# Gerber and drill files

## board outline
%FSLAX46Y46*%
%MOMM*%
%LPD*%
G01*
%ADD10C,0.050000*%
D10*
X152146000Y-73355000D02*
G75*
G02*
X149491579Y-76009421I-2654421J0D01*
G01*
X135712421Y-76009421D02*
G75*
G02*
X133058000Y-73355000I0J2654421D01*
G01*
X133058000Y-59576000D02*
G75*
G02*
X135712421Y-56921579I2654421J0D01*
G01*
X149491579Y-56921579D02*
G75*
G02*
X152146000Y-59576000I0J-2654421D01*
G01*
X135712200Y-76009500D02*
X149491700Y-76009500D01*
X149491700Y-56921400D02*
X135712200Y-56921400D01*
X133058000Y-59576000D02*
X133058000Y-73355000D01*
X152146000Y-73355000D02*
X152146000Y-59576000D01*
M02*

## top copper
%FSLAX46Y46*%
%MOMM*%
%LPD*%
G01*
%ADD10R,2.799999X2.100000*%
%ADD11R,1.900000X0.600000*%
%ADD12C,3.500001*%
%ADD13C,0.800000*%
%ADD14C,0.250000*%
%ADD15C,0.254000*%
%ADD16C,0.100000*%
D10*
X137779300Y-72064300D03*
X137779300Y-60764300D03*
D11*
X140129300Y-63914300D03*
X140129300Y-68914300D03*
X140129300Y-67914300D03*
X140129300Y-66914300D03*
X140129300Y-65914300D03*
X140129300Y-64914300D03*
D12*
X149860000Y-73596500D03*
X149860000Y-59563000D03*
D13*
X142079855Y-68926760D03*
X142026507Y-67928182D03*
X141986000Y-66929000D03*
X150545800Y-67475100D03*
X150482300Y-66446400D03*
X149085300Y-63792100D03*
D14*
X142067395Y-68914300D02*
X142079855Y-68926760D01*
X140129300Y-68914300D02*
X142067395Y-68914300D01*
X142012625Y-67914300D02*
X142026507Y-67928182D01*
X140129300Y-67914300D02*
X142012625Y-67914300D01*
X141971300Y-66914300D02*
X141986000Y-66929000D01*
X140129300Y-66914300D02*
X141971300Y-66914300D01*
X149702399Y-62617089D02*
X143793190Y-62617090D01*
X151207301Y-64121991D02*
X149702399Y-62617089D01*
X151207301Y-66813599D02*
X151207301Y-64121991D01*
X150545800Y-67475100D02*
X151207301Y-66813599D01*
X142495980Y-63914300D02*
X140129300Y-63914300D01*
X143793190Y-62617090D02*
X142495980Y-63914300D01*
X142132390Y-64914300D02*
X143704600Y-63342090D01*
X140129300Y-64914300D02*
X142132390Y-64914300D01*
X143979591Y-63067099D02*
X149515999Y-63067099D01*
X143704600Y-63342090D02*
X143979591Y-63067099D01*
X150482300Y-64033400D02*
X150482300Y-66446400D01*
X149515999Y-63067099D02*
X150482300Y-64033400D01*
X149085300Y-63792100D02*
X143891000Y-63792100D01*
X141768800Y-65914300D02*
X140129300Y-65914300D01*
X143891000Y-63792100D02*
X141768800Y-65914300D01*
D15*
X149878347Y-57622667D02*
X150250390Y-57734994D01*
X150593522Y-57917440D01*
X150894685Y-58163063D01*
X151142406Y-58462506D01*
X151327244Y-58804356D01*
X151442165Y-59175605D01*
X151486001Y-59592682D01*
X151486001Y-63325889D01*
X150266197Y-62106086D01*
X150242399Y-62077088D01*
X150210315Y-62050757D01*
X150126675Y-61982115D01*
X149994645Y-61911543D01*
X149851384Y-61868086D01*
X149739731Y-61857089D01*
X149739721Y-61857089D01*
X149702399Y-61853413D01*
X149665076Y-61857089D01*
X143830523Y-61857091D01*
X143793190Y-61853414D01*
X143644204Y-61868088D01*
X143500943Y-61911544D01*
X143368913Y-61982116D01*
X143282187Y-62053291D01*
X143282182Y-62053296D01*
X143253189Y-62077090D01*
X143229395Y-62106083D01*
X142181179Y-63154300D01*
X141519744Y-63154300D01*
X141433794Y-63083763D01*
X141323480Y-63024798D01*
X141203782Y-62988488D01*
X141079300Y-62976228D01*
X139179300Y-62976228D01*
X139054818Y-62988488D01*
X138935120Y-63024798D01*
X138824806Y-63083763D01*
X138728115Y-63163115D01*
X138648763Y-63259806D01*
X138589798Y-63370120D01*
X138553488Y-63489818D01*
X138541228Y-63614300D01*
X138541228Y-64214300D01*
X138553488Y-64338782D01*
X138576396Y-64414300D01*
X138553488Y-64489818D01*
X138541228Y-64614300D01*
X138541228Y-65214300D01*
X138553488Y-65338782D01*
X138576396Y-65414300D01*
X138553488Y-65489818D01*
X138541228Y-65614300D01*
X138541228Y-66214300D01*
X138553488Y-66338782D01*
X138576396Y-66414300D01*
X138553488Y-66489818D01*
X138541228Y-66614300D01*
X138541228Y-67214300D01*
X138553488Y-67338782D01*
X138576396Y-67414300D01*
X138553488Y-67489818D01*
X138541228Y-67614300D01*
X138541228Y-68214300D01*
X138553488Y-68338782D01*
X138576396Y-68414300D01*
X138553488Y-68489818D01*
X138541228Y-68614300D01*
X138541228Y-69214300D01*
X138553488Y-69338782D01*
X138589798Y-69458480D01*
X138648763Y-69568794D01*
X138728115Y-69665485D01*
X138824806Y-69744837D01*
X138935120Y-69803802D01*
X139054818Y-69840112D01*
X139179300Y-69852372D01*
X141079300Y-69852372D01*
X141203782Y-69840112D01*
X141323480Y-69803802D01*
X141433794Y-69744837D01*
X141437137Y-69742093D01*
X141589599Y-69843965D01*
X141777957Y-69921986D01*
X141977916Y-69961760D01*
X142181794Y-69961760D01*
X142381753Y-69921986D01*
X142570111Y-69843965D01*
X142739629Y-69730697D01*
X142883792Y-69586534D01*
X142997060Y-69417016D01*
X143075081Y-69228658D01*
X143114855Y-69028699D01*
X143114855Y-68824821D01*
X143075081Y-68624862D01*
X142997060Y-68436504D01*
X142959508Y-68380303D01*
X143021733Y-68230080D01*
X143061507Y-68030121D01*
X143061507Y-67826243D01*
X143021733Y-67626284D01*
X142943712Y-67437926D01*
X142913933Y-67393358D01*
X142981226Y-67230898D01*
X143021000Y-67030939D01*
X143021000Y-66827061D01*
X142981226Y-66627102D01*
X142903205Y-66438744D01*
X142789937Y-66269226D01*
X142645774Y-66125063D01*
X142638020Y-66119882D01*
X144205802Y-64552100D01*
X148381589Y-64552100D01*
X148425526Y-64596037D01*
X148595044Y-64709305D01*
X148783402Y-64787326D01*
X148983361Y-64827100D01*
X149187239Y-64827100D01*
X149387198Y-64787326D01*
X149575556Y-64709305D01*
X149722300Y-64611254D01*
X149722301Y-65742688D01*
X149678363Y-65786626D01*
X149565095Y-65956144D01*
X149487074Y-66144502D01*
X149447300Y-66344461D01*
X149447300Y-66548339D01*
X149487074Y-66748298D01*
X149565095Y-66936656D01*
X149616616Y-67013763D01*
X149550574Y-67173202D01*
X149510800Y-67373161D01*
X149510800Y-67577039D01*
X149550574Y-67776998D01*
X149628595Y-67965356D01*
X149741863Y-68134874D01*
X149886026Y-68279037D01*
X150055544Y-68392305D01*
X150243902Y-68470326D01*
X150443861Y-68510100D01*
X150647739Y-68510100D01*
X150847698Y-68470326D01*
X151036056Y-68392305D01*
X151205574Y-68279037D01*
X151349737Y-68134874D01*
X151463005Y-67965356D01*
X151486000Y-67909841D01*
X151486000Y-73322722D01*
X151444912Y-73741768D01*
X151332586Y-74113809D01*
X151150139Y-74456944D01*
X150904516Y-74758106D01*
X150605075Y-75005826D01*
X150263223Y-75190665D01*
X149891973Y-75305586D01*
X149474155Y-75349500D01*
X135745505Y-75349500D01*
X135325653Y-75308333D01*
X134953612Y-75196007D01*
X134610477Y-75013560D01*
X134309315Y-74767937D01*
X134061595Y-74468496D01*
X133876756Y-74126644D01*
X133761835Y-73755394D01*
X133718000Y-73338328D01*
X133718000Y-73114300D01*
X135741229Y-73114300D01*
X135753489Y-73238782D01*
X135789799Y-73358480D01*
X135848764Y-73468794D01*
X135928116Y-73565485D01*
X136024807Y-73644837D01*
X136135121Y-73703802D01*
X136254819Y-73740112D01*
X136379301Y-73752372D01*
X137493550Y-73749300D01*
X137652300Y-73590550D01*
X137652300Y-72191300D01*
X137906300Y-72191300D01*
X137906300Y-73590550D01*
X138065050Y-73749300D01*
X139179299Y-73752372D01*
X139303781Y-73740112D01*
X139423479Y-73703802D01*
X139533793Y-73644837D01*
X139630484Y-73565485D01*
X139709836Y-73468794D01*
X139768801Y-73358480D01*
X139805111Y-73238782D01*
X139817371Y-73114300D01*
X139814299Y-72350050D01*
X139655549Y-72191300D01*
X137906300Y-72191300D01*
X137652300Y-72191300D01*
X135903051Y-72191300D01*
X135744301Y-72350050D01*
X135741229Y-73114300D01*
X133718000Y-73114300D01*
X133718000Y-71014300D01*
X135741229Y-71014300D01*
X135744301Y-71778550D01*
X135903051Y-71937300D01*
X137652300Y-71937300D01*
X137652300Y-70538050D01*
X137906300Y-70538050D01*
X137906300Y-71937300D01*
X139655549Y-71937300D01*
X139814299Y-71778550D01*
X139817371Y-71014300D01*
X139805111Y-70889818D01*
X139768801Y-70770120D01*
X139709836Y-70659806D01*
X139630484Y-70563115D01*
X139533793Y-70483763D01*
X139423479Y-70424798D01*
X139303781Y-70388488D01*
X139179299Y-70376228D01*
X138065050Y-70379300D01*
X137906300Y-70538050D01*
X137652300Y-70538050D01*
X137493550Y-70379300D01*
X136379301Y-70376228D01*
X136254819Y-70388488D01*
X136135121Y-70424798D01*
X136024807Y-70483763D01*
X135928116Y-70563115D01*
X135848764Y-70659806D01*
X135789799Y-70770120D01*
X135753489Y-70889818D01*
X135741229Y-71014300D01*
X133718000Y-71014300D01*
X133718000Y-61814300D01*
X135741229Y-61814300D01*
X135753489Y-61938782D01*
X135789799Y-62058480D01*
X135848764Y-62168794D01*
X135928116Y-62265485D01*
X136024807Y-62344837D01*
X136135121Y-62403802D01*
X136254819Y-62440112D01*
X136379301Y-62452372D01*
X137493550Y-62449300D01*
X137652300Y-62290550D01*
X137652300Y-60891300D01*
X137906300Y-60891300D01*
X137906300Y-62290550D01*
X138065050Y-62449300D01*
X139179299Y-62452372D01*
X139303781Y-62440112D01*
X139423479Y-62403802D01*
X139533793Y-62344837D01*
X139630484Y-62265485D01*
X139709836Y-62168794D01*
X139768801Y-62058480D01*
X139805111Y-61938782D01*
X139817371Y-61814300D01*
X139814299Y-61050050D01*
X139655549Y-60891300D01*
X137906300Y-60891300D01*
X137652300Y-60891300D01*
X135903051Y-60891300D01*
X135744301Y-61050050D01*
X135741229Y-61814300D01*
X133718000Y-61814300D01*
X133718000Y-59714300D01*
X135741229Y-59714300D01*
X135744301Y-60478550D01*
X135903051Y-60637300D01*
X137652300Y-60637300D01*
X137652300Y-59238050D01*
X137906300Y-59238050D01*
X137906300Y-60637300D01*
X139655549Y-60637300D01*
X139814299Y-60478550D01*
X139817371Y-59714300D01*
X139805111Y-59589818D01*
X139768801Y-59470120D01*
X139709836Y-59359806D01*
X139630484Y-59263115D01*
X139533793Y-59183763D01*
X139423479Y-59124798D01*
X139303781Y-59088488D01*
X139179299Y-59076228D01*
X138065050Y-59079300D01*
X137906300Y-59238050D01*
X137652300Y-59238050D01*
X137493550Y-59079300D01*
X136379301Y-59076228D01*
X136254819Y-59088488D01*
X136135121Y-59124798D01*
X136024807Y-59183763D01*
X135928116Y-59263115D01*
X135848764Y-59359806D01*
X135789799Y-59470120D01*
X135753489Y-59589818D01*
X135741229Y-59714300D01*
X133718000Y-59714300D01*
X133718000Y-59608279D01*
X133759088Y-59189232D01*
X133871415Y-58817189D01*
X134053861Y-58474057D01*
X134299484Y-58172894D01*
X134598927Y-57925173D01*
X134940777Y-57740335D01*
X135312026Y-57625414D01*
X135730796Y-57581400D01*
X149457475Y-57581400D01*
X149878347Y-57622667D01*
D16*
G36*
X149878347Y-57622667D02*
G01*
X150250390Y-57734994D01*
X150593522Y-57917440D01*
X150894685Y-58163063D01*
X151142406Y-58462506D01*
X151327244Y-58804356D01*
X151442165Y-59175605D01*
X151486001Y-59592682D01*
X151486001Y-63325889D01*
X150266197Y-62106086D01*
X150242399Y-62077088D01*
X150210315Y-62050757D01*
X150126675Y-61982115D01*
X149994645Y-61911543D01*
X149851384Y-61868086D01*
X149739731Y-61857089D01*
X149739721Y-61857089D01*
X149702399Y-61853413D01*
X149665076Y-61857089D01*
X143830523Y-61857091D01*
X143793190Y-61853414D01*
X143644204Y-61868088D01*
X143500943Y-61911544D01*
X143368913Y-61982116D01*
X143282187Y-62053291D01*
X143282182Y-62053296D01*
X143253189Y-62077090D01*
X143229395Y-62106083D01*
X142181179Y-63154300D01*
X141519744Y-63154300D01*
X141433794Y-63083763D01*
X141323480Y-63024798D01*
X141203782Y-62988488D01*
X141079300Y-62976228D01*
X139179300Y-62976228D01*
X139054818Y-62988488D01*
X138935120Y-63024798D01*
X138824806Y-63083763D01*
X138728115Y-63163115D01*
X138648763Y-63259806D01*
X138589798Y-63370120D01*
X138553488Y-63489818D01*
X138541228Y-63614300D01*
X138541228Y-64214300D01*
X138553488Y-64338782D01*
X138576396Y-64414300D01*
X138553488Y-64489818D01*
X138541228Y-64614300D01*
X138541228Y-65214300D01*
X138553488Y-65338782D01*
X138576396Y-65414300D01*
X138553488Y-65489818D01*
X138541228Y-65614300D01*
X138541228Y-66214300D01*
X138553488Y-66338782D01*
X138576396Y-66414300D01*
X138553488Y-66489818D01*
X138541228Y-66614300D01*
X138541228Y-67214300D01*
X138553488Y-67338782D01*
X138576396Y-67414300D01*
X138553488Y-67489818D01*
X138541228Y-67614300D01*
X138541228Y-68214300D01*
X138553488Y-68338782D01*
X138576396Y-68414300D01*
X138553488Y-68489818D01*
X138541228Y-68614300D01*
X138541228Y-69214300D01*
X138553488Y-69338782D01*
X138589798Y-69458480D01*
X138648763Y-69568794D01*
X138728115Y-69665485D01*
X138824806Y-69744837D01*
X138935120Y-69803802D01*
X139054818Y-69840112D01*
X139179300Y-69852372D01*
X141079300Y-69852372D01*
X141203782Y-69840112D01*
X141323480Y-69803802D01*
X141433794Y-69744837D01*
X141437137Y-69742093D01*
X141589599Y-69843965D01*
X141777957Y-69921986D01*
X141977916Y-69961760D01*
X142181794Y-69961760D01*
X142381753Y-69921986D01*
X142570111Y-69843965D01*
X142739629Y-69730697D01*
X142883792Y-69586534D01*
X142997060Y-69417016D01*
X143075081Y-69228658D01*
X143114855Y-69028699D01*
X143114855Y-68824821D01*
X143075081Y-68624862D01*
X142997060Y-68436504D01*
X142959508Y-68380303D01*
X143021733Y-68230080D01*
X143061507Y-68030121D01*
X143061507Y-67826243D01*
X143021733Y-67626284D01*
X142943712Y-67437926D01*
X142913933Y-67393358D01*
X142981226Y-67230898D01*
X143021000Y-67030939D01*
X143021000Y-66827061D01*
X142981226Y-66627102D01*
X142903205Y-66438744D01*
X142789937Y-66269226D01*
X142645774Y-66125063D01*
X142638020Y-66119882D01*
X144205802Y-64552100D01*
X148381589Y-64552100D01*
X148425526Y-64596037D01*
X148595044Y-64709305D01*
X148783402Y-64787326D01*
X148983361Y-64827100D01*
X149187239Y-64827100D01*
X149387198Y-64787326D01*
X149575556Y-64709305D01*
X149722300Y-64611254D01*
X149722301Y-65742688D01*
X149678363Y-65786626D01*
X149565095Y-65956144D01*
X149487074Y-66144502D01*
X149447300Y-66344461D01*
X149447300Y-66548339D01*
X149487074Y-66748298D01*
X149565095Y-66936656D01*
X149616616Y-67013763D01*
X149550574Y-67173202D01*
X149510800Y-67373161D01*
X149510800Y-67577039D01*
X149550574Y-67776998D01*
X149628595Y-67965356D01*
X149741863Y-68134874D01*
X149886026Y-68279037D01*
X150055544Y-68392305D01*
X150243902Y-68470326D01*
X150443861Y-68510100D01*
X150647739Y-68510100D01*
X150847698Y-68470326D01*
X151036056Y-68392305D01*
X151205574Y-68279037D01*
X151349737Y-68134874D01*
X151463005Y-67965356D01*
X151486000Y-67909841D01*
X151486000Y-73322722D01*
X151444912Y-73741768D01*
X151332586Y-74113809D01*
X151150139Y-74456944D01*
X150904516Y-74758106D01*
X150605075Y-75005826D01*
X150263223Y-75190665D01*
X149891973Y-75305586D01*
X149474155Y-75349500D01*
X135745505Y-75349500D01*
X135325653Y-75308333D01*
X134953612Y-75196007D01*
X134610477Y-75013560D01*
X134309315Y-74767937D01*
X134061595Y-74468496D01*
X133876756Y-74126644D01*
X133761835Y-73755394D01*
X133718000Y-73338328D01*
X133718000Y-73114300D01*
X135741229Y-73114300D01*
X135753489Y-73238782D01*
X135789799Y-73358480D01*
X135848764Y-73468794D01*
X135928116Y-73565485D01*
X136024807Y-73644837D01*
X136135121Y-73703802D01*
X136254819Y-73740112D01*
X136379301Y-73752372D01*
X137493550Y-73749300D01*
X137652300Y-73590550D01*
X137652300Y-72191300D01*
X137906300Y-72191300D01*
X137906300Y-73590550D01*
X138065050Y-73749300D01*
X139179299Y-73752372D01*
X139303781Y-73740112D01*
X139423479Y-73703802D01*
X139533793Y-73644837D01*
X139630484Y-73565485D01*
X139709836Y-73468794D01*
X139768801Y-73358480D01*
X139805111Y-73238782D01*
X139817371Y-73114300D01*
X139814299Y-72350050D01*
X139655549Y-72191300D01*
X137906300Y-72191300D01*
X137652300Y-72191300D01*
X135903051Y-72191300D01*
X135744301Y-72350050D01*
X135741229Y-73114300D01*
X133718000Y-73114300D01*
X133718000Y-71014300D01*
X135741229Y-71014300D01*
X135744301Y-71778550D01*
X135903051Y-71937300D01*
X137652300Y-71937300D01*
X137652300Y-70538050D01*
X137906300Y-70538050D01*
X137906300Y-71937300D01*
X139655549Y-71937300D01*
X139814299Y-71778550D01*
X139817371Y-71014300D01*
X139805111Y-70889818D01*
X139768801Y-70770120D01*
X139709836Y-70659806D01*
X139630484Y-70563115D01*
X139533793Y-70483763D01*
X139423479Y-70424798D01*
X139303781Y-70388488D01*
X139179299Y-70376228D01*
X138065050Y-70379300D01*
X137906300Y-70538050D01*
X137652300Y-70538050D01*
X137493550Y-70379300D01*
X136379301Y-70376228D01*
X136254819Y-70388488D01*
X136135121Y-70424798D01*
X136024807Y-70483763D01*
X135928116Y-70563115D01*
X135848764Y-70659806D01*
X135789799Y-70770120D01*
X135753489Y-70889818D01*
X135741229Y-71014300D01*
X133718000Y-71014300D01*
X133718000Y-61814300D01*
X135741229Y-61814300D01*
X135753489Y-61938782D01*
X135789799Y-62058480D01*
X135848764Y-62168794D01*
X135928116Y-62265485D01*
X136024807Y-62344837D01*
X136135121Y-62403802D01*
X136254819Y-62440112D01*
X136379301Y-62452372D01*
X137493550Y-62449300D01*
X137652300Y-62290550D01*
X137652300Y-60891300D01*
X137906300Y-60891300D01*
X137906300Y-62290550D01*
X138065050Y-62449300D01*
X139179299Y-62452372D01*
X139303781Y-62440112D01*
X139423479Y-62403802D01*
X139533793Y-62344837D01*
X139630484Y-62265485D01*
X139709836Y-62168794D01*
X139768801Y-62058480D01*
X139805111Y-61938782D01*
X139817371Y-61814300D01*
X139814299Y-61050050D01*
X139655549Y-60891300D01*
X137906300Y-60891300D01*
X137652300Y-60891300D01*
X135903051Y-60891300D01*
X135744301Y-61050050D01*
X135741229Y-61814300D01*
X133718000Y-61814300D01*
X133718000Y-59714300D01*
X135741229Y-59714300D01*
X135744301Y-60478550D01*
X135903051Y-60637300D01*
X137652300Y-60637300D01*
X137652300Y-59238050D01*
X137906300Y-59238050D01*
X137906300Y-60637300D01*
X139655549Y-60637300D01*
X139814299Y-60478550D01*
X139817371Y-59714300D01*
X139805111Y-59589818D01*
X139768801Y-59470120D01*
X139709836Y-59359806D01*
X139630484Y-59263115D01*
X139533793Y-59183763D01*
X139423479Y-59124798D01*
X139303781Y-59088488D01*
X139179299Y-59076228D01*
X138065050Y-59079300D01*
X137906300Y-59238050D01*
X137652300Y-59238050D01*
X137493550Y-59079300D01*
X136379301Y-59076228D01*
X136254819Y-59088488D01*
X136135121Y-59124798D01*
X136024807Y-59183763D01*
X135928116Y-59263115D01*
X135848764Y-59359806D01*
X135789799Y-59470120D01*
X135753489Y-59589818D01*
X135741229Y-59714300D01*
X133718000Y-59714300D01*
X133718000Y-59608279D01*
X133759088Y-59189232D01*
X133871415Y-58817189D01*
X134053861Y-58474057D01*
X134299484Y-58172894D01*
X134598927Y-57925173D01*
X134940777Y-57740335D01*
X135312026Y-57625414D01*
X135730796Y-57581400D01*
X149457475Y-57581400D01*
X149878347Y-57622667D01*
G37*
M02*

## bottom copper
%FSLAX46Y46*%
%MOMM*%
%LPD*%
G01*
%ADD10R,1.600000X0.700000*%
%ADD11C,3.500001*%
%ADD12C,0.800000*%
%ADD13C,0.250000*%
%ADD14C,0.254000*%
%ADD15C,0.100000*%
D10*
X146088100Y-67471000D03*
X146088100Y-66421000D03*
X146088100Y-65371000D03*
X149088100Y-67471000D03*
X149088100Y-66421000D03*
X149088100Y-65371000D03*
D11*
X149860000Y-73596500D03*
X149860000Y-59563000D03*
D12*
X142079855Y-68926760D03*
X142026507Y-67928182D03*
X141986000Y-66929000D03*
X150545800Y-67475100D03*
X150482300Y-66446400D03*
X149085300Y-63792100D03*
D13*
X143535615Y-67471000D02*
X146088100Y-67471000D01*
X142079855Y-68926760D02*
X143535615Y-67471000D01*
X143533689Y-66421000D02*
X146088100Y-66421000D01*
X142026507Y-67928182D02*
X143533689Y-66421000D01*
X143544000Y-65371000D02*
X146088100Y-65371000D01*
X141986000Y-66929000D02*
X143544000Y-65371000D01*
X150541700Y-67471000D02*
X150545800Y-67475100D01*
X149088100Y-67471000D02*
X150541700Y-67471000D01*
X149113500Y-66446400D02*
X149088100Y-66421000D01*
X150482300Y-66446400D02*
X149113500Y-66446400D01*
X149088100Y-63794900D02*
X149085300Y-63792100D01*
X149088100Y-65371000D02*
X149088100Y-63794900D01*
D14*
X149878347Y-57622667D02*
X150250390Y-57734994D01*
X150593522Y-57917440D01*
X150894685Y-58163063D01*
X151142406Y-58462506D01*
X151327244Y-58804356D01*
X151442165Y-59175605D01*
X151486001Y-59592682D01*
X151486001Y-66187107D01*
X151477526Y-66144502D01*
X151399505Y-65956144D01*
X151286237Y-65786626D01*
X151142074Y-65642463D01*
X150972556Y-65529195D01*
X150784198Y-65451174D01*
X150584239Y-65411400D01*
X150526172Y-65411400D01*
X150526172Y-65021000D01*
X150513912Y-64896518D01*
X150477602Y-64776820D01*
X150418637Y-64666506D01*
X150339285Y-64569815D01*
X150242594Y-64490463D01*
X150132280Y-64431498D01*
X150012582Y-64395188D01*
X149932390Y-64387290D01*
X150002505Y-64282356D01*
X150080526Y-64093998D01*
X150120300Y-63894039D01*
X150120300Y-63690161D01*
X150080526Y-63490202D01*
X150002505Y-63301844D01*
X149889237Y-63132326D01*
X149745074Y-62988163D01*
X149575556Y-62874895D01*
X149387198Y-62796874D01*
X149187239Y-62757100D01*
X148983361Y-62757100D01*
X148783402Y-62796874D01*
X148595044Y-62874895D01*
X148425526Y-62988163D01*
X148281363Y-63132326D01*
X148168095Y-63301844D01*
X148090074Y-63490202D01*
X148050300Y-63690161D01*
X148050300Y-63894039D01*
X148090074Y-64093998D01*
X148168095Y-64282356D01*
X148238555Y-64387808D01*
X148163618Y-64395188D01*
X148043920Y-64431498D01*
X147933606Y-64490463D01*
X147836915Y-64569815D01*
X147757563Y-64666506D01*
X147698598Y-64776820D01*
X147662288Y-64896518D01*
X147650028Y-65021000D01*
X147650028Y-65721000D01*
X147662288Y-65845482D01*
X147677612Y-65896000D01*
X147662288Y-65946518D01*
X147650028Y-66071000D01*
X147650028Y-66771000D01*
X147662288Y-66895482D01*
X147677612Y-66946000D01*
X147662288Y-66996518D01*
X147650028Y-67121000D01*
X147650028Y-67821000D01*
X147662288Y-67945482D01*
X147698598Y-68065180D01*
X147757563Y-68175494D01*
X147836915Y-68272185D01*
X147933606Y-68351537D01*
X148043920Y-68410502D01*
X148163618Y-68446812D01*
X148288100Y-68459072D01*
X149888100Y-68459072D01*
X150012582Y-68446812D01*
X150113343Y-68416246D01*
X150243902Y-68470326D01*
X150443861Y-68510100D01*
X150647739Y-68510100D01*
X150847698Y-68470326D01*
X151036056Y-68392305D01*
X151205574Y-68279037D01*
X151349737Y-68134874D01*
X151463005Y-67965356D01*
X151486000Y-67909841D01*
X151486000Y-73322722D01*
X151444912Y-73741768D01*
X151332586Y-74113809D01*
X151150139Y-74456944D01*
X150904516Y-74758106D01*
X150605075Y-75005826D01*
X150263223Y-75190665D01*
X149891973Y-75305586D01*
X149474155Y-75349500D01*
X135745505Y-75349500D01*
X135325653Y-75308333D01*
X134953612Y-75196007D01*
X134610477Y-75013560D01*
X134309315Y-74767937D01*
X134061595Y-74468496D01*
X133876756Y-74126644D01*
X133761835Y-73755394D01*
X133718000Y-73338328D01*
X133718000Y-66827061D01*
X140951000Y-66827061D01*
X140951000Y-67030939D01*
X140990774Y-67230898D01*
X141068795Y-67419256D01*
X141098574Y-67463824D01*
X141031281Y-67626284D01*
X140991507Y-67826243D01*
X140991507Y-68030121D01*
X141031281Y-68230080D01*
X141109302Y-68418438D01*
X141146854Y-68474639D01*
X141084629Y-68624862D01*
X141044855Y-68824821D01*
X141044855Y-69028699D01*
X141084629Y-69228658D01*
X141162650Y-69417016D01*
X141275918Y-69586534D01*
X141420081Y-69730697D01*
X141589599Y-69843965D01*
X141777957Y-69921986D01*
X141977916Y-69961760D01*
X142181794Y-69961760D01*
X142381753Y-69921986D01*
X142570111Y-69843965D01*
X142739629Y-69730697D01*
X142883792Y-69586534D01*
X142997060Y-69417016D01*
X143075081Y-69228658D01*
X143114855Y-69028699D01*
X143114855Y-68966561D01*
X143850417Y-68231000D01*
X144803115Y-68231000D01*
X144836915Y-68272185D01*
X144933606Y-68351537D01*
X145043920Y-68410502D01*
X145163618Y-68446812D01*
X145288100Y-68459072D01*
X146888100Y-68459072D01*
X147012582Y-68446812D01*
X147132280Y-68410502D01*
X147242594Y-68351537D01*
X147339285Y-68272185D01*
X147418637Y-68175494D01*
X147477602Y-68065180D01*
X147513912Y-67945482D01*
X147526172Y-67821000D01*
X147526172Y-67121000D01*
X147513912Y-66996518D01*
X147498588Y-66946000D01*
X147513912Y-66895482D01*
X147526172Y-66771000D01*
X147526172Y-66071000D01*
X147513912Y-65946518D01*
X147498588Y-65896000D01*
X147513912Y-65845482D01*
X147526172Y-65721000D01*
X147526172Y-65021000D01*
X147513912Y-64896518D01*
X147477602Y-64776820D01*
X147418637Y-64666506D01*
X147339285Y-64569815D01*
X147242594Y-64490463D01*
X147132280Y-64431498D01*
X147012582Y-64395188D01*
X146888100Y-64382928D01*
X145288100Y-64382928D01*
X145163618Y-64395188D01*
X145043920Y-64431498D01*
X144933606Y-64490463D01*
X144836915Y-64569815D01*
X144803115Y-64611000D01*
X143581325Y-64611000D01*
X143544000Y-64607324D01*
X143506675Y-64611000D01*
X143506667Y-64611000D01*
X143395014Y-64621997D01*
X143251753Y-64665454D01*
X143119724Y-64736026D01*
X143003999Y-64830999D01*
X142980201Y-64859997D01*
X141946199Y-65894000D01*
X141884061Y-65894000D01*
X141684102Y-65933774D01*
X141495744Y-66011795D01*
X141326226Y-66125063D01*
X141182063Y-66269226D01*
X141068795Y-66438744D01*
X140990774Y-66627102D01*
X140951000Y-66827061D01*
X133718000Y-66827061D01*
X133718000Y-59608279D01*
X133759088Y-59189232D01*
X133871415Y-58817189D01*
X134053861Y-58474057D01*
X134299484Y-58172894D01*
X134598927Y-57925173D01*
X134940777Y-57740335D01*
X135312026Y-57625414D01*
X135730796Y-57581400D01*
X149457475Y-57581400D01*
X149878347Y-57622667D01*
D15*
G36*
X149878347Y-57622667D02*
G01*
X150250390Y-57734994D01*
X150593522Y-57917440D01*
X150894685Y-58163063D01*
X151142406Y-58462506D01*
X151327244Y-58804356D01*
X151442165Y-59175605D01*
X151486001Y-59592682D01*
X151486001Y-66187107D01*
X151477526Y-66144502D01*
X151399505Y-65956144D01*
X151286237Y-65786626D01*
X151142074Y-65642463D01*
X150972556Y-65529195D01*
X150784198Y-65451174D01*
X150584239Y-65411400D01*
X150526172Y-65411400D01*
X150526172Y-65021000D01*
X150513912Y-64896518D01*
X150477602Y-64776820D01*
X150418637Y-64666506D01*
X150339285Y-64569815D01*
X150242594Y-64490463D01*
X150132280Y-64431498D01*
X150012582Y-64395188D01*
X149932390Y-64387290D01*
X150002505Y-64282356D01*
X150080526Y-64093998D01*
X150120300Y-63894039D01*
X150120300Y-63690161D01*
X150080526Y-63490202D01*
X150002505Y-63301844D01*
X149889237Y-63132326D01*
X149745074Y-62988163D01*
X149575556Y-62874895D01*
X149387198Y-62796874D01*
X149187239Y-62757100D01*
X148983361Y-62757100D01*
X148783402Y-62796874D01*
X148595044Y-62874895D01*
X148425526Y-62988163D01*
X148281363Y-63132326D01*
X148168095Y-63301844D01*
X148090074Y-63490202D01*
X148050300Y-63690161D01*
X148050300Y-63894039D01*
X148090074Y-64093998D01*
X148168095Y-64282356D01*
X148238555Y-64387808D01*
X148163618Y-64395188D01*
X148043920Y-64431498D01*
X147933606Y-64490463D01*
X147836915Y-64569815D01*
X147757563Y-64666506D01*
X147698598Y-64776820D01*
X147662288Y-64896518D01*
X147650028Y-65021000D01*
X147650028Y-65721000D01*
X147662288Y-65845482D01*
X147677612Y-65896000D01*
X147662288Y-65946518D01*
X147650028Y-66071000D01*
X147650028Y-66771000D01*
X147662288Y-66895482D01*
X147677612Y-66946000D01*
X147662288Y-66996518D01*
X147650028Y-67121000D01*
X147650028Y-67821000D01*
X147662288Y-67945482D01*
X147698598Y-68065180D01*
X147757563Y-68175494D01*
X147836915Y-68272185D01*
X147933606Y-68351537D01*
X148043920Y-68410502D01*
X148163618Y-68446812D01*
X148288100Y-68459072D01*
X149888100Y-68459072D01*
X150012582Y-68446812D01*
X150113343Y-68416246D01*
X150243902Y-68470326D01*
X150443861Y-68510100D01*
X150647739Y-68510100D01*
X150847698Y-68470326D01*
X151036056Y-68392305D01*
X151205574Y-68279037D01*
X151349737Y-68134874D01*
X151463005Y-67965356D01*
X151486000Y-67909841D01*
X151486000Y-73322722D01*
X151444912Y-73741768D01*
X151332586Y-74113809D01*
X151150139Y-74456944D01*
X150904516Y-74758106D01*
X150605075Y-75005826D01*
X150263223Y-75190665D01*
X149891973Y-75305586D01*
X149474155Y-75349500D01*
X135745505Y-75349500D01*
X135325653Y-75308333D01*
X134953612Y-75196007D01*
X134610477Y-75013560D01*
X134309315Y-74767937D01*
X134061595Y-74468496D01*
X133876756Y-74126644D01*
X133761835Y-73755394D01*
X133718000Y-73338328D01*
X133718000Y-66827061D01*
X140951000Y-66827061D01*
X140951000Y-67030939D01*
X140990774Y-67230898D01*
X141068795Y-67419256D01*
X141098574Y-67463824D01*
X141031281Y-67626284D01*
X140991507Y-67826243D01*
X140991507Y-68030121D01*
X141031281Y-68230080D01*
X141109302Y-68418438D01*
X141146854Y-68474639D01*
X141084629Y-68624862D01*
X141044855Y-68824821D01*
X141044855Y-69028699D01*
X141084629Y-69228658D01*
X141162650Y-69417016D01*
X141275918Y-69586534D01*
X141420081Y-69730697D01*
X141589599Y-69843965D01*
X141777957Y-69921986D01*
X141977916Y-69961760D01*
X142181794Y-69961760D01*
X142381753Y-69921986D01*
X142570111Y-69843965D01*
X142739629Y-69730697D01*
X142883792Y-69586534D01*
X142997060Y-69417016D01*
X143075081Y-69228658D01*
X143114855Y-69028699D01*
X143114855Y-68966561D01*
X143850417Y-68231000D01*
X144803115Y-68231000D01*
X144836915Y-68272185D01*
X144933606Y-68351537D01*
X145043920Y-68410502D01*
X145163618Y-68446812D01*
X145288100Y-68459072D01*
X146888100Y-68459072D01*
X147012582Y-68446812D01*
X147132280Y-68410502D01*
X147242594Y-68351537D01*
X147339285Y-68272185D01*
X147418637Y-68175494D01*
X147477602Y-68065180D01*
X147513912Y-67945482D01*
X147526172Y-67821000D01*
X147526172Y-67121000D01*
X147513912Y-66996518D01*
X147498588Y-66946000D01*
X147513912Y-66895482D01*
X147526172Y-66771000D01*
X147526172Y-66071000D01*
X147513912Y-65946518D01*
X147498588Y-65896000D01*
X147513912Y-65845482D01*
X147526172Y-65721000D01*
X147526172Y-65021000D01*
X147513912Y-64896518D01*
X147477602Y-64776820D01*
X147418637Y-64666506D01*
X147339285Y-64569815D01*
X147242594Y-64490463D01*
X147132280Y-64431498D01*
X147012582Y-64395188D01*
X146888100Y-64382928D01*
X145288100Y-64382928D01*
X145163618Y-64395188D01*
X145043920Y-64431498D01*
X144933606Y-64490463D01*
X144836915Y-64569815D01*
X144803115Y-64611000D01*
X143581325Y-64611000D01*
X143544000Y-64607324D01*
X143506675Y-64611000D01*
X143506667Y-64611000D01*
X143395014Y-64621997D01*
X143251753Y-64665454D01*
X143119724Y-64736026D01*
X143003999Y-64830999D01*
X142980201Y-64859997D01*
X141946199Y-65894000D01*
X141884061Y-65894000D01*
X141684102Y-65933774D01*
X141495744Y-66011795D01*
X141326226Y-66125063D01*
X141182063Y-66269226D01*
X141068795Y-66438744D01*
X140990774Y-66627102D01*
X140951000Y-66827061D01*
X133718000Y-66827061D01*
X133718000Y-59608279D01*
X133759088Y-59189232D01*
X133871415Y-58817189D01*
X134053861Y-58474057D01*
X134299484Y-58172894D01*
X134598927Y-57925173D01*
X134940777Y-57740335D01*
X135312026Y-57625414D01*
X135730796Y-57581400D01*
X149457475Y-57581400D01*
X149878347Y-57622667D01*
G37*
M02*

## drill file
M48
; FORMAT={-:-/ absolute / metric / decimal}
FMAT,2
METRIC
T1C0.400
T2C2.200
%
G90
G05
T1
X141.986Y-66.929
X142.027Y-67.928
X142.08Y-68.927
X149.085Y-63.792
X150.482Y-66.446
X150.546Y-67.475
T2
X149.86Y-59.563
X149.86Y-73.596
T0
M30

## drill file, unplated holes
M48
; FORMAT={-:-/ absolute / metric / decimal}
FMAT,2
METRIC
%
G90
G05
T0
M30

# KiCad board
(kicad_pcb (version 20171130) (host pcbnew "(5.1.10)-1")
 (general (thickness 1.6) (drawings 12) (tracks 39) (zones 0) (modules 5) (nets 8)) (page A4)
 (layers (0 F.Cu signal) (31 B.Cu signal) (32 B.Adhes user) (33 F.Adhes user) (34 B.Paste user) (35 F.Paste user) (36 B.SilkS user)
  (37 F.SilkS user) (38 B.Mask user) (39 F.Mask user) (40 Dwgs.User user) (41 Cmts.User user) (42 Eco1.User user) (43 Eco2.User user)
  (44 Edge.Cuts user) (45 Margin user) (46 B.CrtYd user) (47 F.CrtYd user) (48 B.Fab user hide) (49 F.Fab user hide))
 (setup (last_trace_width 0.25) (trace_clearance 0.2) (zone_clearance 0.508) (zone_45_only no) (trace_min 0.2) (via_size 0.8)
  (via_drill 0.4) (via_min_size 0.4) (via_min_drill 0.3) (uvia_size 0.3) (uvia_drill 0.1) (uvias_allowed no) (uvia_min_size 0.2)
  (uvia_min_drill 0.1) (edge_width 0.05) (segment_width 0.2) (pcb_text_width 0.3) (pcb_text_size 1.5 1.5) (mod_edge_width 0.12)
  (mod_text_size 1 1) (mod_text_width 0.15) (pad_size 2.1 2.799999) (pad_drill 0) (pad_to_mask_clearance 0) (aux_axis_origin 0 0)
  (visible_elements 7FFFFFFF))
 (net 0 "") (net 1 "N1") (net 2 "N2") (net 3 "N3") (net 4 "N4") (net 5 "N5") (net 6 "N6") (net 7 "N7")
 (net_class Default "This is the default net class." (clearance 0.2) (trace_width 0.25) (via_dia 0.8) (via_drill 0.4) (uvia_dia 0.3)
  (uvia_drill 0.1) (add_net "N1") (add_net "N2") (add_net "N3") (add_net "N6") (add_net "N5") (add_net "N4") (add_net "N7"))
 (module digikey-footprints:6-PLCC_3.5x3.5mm (layer B.Cu) (at 147.5881 66.421)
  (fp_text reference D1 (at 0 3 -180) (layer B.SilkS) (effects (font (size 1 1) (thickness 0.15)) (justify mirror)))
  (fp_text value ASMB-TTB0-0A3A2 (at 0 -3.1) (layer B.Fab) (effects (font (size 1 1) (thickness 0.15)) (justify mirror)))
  (pad 1 smd rect (at -1.5 1.05) (size 1.6 0.7) (layers B.Cu B.Paste B.Mask) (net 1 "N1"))
  (pad 2 smd rect (at -1.5 0) (size 1.6 0.7) (layers B.Cu B.Paste B.Mask) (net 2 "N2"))
  (pad 3 smd rect (at -1.5 -1.05) (size 1.6 0.7) (layers B.Cu B.Paste B.Mask) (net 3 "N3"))
  (pad 6 smd rect (at 1.5 1.05) (size 1.6 0.7) (layers B.Cu B.Paste B.Mask) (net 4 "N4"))
  (pad 5 smd rect (at 1.5 0) (size 1.6 0.7) (layers B.Cu B.Paste B.Mask) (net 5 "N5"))
  (pad 4 smd rect (at 1.5 -1.05) (size 1.6 0.7) (layers B.Cu B.Paste B.Mask) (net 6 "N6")))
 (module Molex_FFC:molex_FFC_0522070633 (layer F.Cu) (at 139.1793 63.6143 270)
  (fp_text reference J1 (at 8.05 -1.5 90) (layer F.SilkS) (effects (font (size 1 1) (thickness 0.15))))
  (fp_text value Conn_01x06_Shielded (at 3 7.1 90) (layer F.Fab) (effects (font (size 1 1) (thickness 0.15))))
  (pad SH smd rect (at 8.45 1.4 270) (size 2.1 2.799999) (layers F.Cu F.Paste F.Mask) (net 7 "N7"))
  (pad SH smd rect (at -2.85 1.4 270) (size 2.1 2.799999) (layers F.Cu F.Paste F.Mask) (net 7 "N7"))
  (pad 1 smd rect (at 0.3 -0.95 270) (size 0.6 1.9) (layers F.Cu F.Paste F.Mask) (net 4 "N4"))
  (pad 6 smd rect (at 5.3 -0.95 270) (size 0.6 1.9) (layers F.Cu F.Paste F.Mask) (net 1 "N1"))
  (pad 5 smd rect (at 4.3 -0.95 270) (size 0.6 1.9) (layers F.Cu F.Paste F.Mask) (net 2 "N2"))
  (pad 4 smd rect (at 3.3 -0.95 270) (size 0.6 1.9) (layers F.Cu F.Paste F.Mask) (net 3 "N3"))
  (pad 3 smd rect (at 2.3 -0.95 270) (size 0.6 1.9) (layers F.Cu F.Paste F.Mask) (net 6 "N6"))
  (pad 2 smd rect (at 1.3 -0.95 270) (size 0.6 1.9) (layers F.Cu F.Paste F.Mask) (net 5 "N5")))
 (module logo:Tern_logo (layer F.Cu) (at 146.3548 66.2305)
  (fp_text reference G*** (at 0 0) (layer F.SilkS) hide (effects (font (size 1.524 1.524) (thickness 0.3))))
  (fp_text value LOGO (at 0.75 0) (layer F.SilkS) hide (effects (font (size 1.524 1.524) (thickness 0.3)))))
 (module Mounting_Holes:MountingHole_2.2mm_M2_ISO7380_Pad (layer F.Cu) (at 149.86 73.5965)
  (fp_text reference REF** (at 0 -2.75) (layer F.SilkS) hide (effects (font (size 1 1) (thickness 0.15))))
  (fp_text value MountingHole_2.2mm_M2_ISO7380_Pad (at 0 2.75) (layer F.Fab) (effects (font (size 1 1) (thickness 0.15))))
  (pad ~ thru_hole circle (at 0 0) (size 3.500001 3.500001) (drill 2.2) (layers *.Cu *.Mask) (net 7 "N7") (zone_connect 2)))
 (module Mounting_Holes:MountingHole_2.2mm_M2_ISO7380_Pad (layer F.Cu) (at 149.86 59.563)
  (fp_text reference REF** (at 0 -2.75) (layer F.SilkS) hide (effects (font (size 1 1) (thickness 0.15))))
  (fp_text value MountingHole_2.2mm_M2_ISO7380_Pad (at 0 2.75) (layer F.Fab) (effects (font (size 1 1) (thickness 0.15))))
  (pad ~ thru_hole circle (at 0 0) (size 3.500001 3.500001) (drill 2.2) (layers *.Cu *.Mask) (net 7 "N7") (zone_connect 2)))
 (gr_arc (start 149.491579 73.355) (end 149.491579 76.009421) (angle -90) (layer Edge.Cuts) (width 0.05))
 (gr_arc (start 135.712421 73.355) (end 133.058 73.355) (angle -90) (layer Edge.Cuts) (width 0.05))
 (gr_arc (start 135.712421 59.576) (end 135.712421 56.921579) (angle -90) (layer Edge.Cuts) (width 0.05))
 (gr_arc (start 149.491579 59.576) (end 152.146 59.576) (angle -90) (layer Edge.Cuts) (width 0.05))
 (gr_line (start 135.7122 76.0095) (end 149.4917 76.0095) (layer Edge.Cuts) (width 0.05))
 (gr_line (start 149.4917 56.9214) (end 135.7122 56.9214) (layer Edge.Cuts) (width 0.05))
 (gr_line (start 133.058 59.576) (end 133.058 73.355) (layer Edge.Cuts) (width 0.05))
 (gr_line (start 152.146 73.355) (end 152.146 59.576) (layer Edge.Cuts) (width 0.05))
 (via (at 142.079855 68.92676) (size 0.8) (drill 0.4) (layers F.Cu B.Cu) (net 1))
 (segment (start 142.067395 68.9143) (end 142.079855 68.92676) (width 0.25) (layer F.Cu) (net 1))
 (segment (start 140.1293 68.9143) (end 142.067395 68.9143) (width 0.25) (layer F.Cu) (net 1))
 (segment (start 143.535615 67.471) (end 146.0881 67.471) (width 0.25) (layer B.Cu) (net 1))
 (segment (start 142.079855 68.92676) (end 143.535615 67.471) (width 0.25) (layer B.Cu) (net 1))
 (via (at 142.026507 67.928182) (size 0.8) (drill 0.4) (layers F.Cu B.Cu) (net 2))
 (segment (start 142.012625 67.9143) (end 142.026507 67.928182) (width 0.25) (layer F.Cu) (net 2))
 (segment (start 140.1293 67.9143) (end 142.012625 67.9143) (width 0.25) (layer F.Cu) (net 2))
 (segment (start 143.533689 66.421) (end 146.0881 66.421) (width 0.25) (layer B.Cu) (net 2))
 (segment (start 142.026507 67.928182) (end 143.533689 66.421) (width 0.25) (layer B.Cu) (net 2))
 (via (at 141.986 66.929) (size 0.8) (drill 0.4) (layers F.Cu B.Cu) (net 3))
 (segment (start 141.9713 66.9143) (end 141.986 66.929) (width 0.25) (layer F.Cu) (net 3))
 (segment (start 140.1293 66.9143) (end 141.9713 66.9143) (width 0.25) (layer F.Cu) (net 3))
 (segment (start 143.544 65.371) (end 146.0881 65.371) (width 0.25) (layer B.Cu) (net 3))
 (segment (start 141.986 66.929) (end 143.544 65.371) (width 0.25) (layer B.Cu) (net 3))
 (via (at 150.5458 67.4751) (size 0.8) (drill 0.4) (layers F.Cu B.Cu) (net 4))
 (segment (start 150.5417 67.471) (end 150.5458 67.4751) (width 0.25) (layer B.Cu) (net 4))
 (segment (start 149.0881 67.471) (end 150.5417 67.471) (width 0.25) (layer B.Cu) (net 4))
 (segment (start 149.702399 62.617089) (end 143.79319 62.61709) (width 0.25) (layer F.Cu) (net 4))
 (segment (start 151.207301 64.121991) (end 149.702399 62.617089) (width 0.25) (layer F.Cu) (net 4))
 (segment (start 151.207301 66.813599) (end 151.207301 64.121991) (width 0.25) (layer F.Cu) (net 4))
 (segment (start 150.5458 67.4751) (end 151.207301 66.813599) (width 0.25) (layer F.Cu) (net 4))
 (segment (start 142.49598 63.9143) (end 140.1293 63.9143) (width 0.25) (layer F.Cu) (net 4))
 (segment (start 143.79319 62.61709) (end 142.49598 63.9143) (width 0.25) (layer F.Cu) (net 4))
 (segment (start 142.13239 64.9143) (end 143.7046 63.34209) (width 0.25) (layer F.Cu) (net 5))
 (segment (start 140.1293 64.9143) (end 142.13239 64.9143) (width 0.25) (layer F.Cu) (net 5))
 (segment (start 143.979591 63.067099) (end 149.515999 63.067099) (width 0.25) (layer F.Cu) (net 5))
 (segment (start 143.7046 63.34209) (end 143.979591 63.067099) (width 0.25) (layer F.Cu) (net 5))
 (segment (start 150.4823 64.0334) (end 150.4823 66.4464) (width 0.25) (layer F.Cu) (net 5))
 (via (at 150.4823 66.4464) (size 0.8) (drill 0.4) (layers F.Cu B.Cu) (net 5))
 (segment (start 149.515999 63.067099) (end 150.4823 64.0334) (width 0.25) (layer F.Cu) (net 5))
 (segment (start 149.1135 66.4464) (end 149.0881 66.421) (width 0.25) (layer B.Cu) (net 5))
 (segment (start 150.4823 66.4464) (end 149.1135 66.4464) (width 0.25) (layer B.Cu) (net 5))
 (via (at 149.0853 63.7921) (size 0.8) (drill 0.4) (layers F.Cu B.Cu) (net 6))
 (segment (start 149.0881 63.7949) (end 149.0853 63.7921) (width 0.25) (layer B.Cu) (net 6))
 (segment (start 149.0881 65.371) (end 149.0881 63.7949) (width 0.25) (layer B.Cu) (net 6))
 (segment (start 149.0853 63.7921) (end 143.891 63.7921) (width 0.25) (layer F.Cu) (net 6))
 (segment (start 141.7688 65.9143) (end 140.1293 65.9143) (width 0.25) (layer F.Cu) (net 6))
 (segment (start 143.891 63.7921) (end 141.7688 65.9143) (width 0.25) (layer F.Cu) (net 6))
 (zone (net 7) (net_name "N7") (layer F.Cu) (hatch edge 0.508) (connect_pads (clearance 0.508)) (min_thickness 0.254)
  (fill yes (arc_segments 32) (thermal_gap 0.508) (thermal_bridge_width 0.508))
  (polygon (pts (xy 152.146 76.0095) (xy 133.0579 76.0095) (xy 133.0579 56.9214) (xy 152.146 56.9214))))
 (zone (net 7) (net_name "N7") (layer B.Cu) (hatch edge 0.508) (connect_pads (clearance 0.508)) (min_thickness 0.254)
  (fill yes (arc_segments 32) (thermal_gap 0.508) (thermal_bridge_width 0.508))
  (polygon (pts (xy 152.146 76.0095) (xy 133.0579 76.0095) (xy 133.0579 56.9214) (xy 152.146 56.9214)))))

